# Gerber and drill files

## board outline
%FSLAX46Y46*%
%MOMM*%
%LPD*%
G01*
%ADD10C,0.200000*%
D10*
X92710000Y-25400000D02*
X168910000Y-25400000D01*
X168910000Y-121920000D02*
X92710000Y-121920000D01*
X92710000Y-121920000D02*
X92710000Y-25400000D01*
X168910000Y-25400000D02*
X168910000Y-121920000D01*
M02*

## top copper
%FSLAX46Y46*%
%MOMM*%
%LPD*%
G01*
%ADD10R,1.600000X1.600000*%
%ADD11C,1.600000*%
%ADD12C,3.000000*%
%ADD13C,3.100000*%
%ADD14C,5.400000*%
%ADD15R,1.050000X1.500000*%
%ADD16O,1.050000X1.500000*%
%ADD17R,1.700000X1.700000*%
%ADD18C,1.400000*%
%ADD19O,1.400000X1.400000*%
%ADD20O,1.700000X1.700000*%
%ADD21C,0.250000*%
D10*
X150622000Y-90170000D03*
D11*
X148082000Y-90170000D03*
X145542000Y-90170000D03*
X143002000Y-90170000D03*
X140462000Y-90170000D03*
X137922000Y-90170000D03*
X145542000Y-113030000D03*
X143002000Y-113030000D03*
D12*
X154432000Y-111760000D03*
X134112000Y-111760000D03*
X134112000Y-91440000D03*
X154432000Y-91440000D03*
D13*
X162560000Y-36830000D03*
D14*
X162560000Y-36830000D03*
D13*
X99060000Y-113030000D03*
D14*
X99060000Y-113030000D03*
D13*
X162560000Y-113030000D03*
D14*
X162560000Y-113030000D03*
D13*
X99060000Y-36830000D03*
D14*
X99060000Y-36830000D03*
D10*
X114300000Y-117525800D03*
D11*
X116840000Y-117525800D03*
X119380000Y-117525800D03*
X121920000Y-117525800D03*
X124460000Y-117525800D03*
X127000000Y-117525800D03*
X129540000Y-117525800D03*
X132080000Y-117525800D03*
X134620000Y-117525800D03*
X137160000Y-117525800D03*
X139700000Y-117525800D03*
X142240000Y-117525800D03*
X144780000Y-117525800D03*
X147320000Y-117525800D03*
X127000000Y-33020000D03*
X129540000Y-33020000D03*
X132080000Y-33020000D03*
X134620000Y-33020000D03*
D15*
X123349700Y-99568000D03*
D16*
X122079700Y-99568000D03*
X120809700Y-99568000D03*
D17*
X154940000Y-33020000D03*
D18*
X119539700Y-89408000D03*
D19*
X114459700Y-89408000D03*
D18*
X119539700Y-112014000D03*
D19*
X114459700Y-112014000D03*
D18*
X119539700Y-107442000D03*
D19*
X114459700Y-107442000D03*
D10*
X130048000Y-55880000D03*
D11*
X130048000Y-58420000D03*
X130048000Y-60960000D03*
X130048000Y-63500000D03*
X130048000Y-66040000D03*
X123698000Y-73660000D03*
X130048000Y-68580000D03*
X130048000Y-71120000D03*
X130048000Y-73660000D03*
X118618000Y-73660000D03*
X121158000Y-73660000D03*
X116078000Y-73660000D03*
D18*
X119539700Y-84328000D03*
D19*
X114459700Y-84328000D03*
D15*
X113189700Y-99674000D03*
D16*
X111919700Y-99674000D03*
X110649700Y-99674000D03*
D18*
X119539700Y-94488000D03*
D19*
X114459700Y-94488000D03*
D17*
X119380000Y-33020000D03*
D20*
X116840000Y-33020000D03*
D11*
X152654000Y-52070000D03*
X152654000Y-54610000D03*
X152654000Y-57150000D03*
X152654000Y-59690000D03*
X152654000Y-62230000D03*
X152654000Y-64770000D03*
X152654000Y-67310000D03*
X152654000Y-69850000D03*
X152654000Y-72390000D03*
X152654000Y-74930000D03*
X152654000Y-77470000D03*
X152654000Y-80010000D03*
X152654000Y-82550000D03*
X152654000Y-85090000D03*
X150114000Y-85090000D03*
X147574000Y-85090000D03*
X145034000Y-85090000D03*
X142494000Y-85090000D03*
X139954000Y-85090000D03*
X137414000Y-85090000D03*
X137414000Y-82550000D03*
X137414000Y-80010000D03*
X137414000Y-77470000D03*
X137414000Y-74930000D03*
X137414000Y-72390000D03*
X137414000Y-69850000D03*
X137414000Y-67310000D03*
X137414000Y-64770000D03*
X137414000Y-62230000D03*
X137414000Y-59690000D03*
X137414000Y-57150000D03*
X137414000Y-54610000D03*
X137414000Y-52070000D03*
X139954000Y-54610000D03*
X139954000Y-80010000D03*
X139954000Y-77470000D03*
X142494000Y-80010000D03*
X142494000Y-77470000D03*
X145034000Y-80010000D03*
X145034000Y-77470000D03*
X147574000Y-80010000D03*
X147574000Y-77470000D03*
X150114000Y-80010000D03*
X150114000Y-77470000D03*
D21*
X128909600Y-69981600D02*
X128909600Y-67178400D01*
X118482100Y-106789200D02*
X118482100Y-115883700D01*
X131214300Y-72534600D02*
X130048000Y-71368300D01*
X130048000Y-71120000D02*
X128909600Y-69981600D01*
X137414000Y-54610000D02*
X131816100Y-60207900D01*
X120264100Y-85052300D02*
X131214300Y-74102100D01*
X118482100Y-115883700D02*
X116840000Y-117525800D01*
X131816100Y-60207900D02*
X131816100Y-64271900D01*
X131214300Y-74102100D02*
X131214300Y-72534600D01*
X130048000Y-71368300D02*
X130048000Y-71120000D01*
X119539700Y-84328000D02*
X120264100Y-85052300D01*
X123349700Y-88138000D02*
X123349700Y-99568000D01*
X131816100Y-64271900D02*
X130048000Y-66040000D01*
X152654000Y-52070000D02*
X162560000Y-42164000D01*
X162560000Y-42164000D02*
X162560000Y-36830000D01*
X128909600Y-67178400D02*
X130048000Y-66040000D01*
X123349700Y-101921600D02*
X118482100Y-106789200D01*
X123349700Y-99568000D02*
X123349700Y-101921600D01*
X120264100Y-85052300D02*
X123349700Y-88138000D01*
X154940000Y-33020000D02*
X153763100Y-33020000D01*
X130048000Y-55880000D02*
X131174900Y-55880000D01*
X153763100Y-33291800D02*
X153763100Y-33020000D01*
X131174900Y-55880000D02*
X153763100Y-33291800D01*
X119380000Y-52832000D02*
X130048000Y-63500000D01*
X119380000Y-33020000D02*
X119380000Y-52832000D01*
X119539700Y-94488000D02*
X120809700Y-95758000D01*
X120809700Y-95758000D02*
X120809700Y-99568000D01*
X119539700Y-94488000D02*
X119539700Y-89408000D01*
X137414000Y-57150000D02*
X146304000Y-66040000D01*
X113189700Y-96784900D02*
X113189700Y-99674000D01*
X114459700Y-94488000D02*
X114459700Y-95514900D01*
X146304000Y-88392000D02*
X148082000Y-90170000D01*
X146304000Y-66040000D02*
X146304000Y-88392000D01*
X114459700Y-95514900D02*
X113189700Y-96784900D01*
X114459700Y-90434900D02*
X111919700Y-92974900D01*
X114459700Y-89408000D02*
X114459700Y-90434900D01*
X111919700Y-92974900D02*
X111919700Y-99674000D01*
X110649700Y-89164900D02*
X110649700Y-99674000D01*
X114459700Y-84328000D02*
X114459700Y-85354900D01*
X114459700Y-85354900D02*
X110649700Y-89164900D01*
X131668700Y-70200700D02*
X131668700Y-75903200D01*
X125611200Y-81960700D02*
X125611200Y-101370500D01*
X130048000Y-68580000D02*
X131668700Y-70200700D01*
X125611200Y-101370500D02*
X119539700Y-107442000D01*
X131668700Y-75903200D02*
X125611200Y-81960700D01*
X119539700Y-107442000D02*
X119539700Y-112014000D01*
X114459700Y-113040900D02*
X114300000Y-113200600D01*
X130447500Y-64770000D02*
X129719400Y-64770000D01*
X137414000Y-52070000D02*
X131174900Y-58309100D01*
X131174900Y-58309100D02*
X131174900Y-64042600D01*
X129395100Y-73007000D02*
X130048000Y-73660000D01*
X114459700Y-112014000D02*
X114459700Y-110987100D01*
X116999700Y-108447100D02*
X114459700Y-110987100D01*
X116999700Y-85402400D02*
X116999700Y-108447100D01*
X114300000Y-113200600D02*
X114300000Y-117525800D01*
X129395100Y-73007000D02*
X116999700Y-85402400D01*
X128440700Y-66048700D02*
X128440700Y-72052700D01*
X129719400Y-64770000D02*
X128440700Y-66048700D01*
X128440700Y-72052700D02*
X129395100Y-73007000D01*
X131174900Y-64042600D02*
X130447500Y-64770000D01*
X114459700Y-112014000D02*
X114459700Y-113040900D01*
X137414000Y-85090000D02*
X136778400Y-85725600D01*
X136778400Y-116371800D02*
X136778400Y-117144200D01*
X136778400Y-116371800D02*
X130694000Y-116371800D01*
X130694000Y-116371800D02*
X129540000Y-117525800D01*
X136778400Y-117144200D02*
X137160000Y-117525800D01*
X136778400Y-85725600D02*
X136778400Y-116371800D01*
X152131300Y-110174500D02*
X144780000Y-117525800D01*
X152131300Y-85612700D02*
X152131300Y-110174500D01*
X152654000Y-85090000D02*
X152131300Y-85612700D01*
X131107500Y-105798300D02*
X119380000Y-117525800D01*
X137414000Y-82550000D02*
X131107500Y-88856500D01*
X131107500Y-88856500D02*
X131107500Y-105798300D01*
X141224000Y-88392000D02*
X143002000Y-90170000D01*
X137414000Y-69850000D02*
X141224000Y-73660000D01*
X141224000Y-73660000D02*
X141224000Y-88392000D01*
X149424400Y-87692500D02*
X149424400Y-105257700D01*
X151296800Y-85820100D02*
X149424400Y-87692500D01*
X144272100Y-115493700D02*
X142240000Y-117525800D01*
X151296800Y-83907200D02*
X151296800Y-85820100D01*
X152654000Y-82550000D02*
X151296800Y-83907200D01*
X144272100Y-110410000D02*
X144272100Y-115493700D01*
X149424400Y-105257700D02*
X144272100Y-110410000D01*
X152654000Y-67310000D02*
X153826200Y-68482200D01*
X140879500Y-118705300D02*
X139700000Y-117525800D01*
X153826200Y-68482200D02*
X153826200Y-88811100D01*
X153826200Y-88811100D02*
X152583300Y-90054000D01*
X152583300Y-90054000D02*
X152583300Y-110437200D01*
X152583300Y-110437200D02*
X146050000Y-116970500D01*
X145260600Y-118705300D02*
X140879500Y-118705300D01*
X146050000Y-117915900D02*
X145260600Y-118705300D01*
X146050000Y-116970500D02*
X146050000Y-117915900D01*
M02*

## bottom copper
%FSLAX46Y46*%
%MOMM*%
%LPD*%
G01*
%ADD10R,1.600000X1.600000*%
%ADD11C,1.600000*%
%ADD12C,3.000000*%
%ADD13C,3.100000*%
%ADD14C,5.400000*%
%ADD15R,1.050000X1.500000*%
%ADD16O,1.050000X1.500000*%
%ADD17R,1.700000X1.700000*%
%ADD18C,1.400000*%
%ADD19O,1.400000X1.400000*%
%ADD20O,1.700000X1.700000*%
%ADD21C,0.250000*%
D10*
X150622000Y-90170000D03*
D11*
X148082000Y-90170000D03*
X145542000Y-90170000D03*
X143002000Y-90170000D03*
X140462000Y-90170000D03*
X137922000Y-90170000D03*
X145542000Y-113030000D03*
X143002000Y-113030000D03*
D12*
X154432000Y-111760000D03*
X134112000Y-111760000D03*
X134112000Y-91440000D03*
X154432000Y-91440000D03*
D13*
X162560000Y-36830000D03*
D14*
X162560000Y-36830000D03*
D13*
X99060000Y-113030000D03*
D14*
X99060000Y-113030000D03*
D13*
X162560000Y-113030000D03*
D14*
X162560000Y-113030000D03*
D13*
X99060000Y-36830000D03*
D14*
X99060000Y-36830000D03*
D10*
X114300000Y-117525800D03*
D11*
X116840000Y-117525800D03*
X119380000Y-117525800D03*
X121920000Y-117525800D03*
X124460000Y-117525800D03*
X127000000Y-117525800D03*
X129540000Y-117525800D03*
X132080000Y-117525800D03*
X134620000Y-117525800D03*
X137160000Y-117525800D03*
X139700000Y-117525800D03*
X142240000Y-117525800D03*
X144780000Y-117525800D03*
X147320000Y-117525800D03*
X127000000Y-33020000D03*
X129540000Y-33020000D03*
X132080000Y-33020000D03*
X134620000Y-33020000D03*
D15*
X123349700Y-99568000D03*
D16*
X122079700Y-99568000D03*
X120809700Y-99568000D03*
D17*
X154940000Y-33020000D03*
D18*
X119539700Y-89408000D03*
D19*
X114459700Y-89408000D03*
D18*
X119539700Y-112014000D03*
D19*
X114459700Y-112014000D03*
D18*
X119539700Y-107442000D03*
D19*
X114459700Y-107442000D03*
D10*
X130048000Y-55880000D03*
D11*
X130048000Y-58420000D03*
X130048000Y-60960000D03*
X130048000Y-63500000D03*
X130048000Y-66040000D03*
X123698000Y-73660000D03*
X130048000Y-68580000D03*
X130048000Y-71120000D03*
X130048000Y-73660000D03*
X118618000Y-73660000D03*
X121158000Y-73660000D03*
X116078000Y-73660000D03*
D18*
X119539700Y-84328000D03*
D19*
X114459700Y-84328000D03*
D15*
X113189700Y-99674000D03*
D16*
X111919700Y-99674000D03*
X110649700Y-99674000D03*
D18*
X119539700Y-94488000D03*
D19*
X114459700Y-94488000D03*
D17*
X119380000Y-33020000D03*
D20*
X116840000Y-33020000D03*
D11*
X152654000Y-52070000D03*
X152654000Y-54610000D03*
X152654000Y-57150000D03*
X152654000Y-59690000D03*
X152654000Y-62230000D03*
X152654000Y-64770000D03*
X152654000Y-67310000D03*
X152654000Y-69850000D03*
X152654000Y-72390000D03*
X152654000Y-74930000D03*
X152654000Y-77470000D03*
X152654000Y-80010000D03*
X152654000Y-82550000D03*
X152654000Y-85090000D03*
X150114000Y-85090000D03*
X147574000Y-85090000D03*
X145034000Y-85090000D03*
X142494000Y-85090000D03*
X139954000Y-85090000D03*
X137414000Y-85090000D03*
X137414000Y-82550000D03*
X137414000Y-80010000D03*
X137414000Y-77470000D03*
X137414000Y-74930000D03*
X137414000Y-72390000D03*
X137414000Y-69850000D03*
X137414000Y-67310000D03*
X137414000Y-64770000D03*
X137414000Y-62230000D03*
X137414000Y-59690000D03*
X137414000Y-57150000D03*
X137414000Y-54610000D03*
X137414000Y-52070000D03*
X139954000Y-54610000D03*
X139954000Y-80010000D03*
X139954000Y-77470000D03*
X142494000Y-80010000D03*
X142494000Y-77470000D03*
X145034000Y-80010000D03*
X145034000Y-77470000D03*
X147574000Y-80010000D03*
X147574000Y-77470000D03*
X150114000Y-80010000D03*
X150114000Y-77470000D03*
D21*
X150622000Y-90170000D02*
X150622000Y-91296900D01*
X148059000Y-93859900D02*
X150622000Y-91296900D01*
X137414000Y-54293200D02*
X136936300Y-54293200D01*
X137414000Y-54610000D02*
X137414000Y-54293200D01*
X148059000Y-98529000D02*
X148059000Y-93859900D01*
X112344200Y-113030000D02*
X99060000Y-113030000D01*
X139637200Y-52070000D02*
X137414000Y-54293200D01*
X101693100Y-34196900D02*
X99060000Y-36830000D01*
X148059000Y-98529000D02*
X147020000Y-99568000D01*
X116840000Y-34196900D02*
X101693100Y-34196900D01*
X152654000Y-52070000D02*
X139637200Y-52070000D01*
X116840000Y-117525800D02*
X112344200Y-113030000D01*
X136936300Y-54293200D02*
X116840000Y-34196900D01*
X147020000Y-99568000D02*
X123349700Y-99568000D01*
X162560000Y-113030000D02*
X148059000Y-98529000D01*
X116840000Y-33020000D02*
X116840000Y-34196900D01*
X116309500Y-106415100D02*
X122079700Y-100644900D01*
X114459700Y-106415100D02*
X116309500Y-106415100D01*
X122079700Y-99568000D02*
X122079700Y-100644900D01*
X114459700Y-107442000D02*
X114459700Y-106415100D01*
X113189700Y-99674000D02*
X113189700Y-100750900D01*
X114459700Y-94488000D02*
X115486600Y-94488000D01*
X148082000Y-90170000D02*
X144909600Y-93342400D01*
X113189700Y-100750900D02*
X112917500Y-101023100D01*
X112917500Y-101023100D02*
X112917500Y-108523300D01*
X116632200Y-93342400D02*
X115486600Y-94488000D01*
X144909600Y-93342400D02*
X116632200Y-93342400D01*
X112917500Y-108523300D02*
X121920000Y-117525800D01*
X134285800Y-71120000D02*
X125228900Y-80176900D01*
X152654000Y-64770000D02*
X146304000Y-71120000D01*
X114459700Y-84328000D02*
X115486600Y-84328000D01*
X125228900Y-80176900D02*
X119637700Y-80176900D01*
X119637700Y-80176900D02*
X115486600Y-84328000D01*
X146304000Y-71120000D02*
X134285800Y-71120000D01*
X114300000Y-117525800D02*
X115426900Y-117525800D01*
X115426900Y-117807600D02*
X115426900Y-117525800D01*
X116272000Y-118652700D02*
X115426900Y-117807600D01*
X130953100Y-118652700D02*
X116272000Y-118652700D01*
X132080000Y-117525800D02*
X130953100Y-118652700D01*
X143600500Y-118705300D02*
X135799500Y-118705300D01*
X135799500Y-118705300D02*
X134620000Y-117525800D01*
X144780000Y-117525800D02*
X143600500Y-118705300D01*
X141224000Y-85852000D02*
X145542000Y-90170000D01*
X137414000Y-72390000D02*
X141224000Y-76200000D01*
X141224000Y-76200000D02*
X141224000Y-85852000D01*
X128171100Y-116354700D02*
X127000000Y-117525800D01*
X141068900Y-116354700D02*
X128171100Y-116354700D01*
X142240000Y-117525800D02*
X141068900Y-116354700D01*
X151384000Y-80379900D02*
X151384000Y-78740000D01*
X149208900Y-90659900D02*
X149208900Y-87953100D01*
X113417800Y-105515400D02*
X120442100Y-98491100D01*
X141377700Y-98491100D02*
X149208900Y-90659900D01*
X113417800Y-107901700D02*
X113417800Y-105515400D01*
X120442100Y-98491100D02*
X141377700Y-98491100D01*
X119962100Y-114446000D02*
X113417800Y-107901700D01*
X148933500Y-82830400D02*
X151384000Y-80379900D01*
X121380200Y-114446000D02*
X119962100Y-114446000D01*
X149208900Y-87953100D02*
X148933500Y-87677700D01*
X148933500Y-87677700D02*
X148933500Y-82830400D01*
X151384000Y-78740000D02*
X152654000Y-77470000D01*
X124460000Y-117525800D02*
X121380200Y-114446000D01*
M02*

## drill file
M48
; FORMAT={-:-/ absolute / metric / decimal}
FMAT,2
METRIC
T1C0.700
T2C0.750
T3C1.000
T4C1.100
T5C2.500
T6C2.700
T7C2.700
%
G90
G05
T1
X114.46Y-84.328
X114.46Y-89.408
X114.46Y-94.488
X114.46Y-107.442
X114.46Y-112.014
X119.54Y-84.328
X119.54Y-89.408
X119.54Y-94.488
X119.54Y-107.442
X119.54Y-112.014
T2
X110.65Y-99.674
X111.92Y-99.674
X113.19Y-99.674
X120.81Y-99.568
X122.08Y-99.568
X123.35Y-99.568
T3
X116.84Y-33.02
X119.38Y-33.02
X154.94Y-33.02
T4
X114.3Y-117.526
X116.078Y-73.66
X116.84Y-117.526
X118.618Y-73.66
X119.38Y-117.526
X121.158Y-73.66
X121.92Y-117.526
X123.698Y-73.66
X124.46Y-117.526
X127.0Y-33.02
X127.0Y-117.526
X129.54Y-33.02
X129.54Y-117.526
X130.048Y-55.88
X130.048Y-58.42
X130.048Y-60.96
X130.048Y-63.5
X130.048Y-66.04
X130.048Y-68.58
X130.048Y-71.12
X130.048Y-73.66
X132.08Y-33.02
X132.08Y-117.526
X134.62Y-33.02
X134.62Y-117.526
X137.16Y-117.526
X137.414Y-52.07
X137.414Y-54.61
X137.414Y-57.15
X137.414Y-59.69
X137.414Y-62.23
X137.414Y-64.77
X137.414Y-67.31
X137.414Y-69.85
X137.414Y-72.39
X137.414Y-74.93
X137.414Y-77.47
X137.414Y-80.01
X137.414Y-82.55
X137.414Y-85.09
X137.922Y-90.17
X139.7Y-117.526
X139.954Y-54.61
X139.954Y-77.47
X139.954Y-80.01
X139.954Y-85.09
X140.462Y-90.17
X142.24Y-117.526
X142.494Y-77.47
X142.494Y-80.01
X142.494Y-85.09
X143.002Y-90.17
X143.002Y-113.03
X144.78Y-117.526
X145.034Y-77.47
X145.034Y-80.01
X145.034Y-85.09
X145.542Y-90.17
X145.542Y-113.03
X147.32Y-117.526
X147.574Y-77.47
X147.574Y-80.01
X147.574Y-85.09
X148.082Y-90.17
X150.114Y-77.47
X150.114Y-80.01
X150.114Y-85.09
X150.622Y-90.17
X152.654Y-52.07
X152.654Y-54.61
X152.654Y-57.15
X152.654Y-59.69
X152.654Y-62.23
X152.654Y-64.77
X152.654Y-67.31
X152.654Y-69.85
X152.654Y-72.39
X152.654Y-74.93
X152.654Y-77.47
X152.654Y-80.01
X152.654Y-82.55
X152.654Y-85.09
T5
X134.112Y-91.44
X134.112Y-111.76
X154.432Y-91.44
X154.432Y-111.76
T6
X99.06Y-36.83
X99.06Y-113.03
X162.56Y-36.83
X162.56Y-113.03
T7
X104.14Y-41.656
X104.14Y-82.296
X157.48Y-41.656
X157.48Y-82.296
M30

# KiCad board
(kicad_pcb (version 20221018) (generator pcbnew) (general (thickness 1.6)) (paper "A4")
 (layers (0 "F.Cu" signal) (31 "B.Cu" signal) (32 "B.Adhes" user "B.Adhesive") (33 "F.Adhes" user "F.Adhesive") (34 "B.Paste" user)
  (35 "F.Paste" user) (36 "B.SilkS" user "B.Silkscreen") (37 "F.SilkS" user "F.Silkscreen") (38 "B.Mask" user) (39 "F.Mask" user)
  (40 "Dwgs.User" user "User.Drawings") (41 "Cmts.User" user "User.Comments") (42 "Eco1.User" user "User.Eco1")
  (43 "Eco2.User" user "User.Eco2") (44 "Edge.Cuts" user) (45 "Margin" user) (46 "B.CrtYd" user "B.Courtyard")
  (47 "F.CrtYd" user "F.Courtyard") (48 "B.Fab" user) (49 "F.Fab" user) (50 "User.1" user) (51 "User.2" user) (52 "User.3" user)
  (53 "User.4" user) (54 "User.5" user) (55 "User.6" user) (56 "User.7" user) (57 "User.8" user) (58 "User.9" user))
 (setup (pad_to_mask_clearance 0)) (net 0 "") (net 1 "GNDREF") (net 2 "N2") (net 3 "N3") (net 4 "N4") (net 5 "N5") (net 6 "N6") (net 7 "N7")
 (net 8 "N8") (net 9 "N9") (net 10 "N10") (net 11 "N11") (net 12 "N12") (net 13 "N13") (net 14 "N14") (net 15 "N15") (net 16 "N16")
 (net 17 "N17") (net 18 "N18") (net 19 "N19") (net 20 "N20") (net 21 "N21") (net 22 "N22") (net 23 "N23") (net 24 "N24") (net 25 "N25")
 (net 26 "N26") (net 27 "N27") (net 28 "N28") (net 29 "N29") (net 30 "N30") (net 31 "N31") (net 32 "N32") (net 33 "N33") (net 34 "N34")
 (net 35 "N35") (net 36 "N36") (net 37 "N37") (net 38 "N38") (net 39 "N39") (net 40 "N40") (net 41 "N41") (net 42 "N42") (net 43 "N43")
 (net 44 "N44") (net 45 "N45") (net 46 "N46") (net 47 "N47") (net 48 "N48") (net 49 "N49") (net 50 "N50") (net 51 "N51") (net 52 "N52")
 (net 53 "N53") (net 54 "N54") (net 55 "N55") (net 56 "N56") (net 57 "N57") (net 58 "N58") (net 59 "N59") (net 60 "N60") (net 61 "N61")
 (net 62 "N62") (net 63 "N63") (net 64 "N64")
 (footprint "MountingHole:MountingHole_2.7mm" (layer "F.Cu") (at 157.48 41.656)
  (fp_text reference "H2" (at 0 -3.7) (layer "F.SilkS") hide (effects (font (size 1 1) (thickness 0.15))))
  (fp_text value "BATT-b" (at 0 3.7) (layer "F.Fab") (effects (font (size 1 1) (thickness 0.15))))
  (pad "" np_thru_hole circle (at 0 0) (size 2.7 2.7) (drill 2.7) (layers "*.Cu" "*.Mask")))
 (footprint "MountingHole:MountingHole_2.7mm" (layer "F.Cu") (at 157.48 82.296)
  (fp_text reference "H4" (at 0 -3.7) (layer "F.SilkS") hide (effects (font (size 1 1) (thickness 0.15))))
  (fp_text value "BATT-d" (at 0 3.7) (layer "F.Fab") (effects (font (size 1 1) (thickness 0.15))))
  (pad "" np_thru_hole circle (at 0 0) (size 2.7 2.7) (drill 2.7) (layers "*.Cu" "*.Mask")))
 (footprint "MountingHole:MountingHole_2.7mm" (layer "F.Cu") (at 104.14 82.296)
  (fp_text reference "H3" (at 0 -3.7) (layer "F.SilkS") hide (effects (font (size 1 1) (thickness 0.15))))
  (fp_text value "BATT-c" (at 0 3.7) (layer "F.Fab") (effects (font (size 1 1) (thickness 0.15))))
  (pad "" np_thru_hole circle (at 0 0) (size 2.7 2.7) (drill 2.7) (layers "*.Cu" "*.Mask")))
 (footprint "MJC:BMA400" (layer "F.Cu") (at 144.272 101.6 180)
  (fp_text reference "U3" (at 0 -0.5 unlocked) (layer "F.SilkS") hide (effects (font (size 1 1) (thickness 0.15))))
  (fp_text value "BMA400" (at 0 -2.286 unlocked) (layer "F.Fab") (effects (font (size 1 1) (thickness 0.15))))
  (pad "1" thru_hole rect (at -6.35 11.43 180) (size 1.6 1.6) (drill 1.1) (layers "*.Cu" "*.Mask") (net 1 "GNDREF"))
  (pad "2" thru_hole circle (at -3.81 11.43 180) (size 1.6 1.6) (drill 1.1) (layers "*.Cu" "*.Mask") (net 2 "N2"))
  (pad "3" thru_hole circle (at -1.27 11.43 180) (size 1.6 1.6) (drill 1.1) (layers "*.Cu" "*.Mask") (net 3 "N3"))
  (pad "4" thru_hole circle (at 1.27 11.43 180) (size 1.6 1.6) (drill 1.1) (layers "*.Cu" "*.Mask") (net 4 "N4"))
  (pad "5" thru_hole circle (at 3.81 11.43 180) (size 1.6 1.6) (drill 1.1) (layers "*.Cu" "*.Mask") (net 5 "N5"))
  (pad "6" thru_hole circle (at 6.35 11.43 180) (size 1.6 1.6) (drill 1.1) (layers "*.Cu" "*.Mask") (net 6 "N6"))
  (pad "7" thru_hole circle (at -1.27 -11.43 180) (size 1.6 1.6) (drill 1.1) (layers "*.Cu" "*.Mask") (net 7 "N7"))
  (pad "8" thru_hole circle (at 1.27 -11.43 180) (size 1.6 1.6) (drill 1.1) (layers "*.Cu" "*.Mask") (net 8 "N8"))
  (pad "9" thru_hole circle (at -10.16 -10.16 180) (size 3 3) (drill 2.5) (layers "*.Cu" "*.Mask"))
  (pad "10" thru_hole circle (at 10.16 -10.16 180) (size 3 3) (drill 2.5) (layers "*.Cu" "*.Mask"))
  (pad "11" thru_hole circle (at 10.16 10.16 180) (size 3 3) (drill 2.5) (layers "*.Cu" "*.Mask"))
  (pad "12" thru_hole circle (at -10.16 10.16 180) (size 3 3) (drill 2.5) (layers "*.Cu" "*.Mask")))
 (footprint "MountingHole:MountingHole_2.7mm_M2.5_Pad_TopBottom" (layer "F.Cu") (at 162.56 36.83)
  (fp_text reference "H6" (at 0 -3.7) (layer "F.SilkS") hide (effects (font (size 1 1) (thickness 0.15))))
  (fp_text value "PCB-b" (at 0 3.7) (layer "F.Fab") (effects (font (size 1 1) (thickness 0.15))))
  (pad "1" thru_hole circle (at 0 0) (size 3.1 3.1) (drill 2.7) (layers "*.Cu" "*.Mask") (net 1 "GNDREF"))
  (pad "1" connect circle (at 0 0) (size 5.4 5.4) (layers "F.Cu" "F.Mask") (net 1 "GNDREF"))
  (pad "1" connect circle (at 0 0) (size 5.4 5.4) (layers "B.Cu" "B.Mask") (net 1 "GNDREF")))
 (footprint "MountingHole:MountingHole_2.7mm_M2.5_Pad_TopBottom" (layer "F.Cu") (at 99.06 113.03)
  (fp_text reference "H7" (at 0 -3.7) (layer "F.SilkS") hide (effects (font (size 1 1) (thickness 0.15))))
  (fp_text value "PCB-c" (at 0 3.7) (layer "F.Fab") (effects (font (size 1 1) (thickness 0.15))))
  (pad "1" thru_hole circle (at 0 0) (size 3.1 3.1) (drill 2.7) (layers "*.Cu" "*.Mask") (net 1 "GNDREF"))
  (pad "1" connect circle (at 0 0) (size 5.4 5.4) (layers "F.Cu" "F.Mask") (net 1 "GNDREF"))
  (pad "1" connect circle (at 0 0) (size 5.4 5.4) (layers "B.Cu" "B.Mask") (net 1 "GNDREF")))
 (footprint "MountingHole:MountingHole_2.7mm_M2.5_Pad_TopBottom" (layer "F.Cu") (at 162.56 113.03)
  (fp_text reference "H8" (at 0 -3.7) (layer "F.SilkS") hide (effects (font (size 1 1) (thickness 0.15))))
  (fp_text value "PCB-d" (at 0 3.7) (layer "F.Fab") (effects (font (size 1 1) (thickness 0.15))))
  (pad "1" thru_hole circle (at 0 0) (size 3.1 3.1) (drill 2.7) (layers "*.Cu" "*.Mask") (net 1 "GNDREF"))
  (pad "1" connect circle (at 0 0) (size 5.4 5.4) (layers "F.Cu" "F.Mask") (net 1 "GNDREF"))
  (pad "1" connect circle (at 0 0) (size 5.4 5.4) (layers "B.Cu" "B.Mask") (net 1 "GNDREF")))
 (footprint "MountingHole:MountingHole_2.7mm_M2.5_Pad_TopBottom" (layer "F.Cu") (at 99.06 36.83)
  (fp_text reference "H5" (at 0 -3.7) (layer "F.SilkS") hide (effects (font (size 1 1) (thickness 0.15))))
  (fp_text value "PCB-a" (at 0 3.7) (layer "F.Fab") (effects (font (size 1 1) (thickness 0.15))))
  (pad "1" thru_hole circle (at 0 0) (size 3.1 3.1) (drill 2.7) (layers "*.Cu" "*.Mask") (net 1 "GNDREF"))
  (pad "1" connect circle (at 0 0) (size 5.4 5.4) (layers "F.Cu" "F.Mask") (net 1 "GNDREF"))
  (pad "1" connect circle (at 0 0) (size 5.4 5.4) (layers "B.Cu" "B.Mask") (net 1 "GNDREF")))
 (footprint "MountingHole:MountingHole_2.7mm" (layer "F.Cu") (at 104.14 41.656)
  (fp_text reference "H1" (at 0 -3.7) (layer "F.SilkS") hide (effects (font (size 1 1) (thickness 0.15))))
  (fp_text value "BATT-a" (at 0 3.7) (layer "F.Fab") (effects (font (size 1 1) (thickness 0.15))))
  (pad "" np_thru_hole circle (at 0 0) (size 2.7 2.7) (drill 2.7) (layers "*.Cu" "*.Mask")))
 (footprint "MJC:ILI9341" (layer "F.Cu") (at 130.81 74.7776)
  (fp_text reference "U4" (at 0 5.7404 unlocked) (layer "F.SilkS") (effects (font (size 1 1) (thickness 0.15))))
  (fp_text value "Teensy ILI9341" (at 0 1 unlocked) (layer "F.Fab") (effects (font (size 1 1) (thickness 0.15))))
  (pad "1" thru_hole rect (at -16.51 42.7482) (size 1.6 1.6) (drill 1.1) (layers "*.Cu" "*.Mask") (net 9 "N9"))
  (pad "2" thru_hole circle (at -13.97 42.7482) (size 1.6 1.6) (drill 1.1) (layers "*.Cu" "*.Mask") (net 1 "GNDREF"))
  (pad "3" thru_hole circle (at -11.43 42.7482) (size 1.6 1.6) (drill 1.1) (layers "*.Cu" "*.Mask") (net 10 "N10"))
  (pad "4" thru_hole circle (at -8.89 42.7482) (size 1.6 1.6) (drill 1.1) (layers "*.Cu" "*.Mask") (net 2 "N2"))
  (pad "5" thru_hole circle (at -6.35 42.7482) (size 1.6 1.6) (drill 1.1) (layers "*.Cu" "*.Mask") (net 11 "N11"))
  (pad "6" thru_hole circle (at -3.81 42.7482) (size 1.6 1.6) (drill 1.1) (layers "*.Cu" "*.Mask") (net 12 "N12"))
  (pad "7" thru_hole circle (at -1.27 42.7482) (size 1.6 1.6) (drill 1.1) (layers "*.Cu" "*.Mask") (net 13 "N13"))
  (pad "8" thru_hole circle (at 1.27 42.7482) (size 1.6 1.6) (drill 1.1) (layers "*.Cu" "*.Mask") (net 9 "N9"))
  (pad "9" thru_hole circle (at 3.81 42.7482) (size 1.6 1.6) (drill 1.1) (layers "*.Cu" "*.Mask") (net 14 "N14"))
  (pad "10" thru_hole circle (at 6.35 42.7482) (size 1.6 1.6) (drill 1.1) (layers "*.Cu" "*.Mask") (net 13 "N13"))
  (pad "11" thru_hole circle (at 8.89 42.7482) (size 1.6 1.6) (drill 1.1) (layers "*.Cu" "*.Mask") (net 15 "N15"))
  (pad "12" thru_hole circle (at 11.43 42.7482) (size 1.6 1.6) (drill 1.1) (layers "*.Cu" "*.Mask") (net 12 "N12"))
  (pad "13" thru_hole circle (at 13.97 42.7482) (size 1.6 1.6) (drill 1.1) (layers "*.Cu" "*.Mask") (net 14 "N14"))
  (pad "14" thru_hole circle (at 16.51 42.7482) (size 1.6 1.6) (drill 1.1) (layers "*.Cu" "*.Mask") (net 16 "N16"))
  (pad "15" thru_hole circle (at -3.81 -41.7576) (size 1.6 1.6) (drill 1.1) (layers "*.Cu" "*.Mask") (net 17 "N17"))
  (pad "16" thru_hole circle (at -1.27 -41.7576) (size 1.6 1.6) (drill 1.1) (layers "*.Cu" "*.Mask") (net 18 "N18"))
  (pad "17" thru_hole circle (at 1.27 -41.7576) (size 1.6 1.6) (drill 1.1) (layers "*.Cu" "*.Mask") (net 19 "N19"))
  (pad "18" thru_hole circle (at 3.81 -41.7576) (size 1.6 1.6) (drill 1.1) (layers "*.Cu" "*.Mask") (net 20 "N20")))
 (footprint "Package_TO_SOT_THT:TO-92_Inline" (layer "B.Cu") (at 123.3497 99.568 180)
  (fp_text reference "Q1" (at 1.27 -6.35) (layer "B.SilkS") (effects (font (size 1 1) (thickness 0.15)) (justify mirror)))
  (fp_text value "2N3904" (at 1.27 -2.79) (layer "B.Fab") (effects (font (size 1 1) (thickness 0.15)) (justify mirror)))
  (pad "1" thru_hole rect (at 0 0 180) (size 1.05 1.5) (drill 0.75) (layers "*.Cu" "*.Mask") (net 1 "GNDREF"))
  (pad "2" thru_hole oval (at 1.27 0 180) (size 1.05 1.5) (drill 0.75) (layers "*.Cu" "*.Mask") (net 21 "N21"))
  (pad "3" thru_hole oval (at 2.54 0 180) (size 1.05 1.5) (drill 0.75) (layers "*.Cu" "*.Mask") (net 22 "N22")))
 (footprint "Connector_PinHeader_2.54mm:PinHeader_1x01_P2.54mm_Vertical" (layer "B.Cu") (at 154.94 33.02 180)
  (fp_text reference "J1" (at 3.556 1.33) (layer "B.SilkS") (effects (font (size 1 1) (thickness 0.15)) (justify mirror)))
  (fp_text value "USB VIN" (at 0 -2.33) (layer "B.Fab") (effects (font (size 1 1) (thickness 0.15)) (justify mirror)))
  (pad "1" thru_hole rect (at 0 0 180) (size 1.7 1.7) (drill 1) (layers "*.Cu" "*.Mask") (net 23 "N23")))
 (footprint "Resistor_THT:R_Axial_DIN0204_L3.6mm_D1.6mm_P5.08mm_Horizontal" (layer "B.Cu") (at 119.5397 89.408 180)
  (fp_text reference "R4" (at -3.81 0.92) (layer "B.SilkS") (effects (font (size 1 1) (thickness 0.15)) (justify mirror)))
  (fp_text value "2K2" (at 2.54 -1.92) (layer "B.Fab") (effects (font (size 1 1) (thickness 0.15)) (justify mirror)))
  (pad "1" thru_hole circle (at 0 0 180) (size 1.4 1.4) (drill 0.7) (layers "*.Cu" "*.Mask") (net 22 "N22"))
  (pad "2" thru_hole oval (at 5.08 0 180) (size 1.4 1.4) (drill 0.7) (layers "*.Cu" "*.Mask") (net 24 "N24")))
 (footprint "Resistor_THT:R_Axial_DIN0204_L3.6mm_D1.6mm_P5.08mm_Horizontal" (layer "B.Cu") (at 119.5397 112.014 180)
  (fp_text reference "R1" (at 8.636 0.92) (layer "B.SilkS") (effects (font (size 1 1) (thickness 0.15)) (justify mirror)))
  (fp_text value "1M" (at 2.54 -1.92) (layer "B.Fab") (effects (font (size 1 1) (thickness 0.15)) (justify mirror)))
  (pad "1" thru_hole circle (at 0 0 180) (size 1.4 1.4) (drill 0.7) (layers "*.Cu" "*.Mask") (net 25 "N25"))
  (pad "2" thru_hole oval (at 5.08 0 180) (size 1.4 1.4) (drill 0.7) (layers "*.Cu" "*.Mask") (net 9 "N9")))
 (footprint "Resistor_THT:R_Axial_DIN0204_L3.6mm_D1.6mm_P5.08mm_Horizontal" (layer "B.Cu") (at 119.5397 107.442 180)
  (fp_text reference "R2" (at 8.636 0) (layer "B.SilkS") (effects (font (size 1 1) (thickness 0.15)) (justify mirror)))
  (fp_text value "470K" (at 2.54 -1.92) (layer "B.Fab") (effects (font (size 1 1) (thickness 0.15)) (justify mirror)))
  (pad "1" thru_hole circle (at 0 0 180) (size 1.4 1.4) (drill 0.7) (layers "*.Cu" "*.Mask") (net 25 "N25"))
  (pad "2" thru_hole oval (at 5.08 0 180) (size 1.4 1.4) (drill 0.7) (layers "*.Cu" "*.Mask") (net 21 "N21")))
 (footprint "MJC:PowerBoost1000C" (layer "B.Cu") (at 119.888 60.96 180)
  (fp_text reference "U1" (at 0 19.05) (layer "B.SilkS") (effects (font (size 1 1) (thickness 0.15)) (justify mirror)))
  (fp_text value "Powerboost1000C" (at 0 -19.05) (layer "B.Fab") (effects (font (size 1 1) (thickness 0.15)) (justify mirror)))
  (pad "1" thru_hole rect (at -10.16 5.08 180) (size 1.6 1.6) (drill 1.1) (layers "*.Cu" "*.Mask") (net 23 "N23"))
  (pad "2" thru_hole circle (at -10.16 2.54 180) (size 1.6 1.6) (drill 1.1) (layers "*.Cu" "*.Mask") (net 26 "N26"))
  (pad "3" thru_hole circle (at -10.16 0 180) (size 1.6 1.6) (drill 1.1) (layers "*.Cu" "*.Mask") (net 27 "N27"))
  (pad "4" thru_hole circle (at -10.16 -2.54 180) (size 1.6 1.6) (drill 1.1) (layers "*.Cu" "*.Mask") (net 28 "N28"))
  (pad "5" thru_hole circle (at -10.16 -5.08 180) (size 1.6 1.6) (drill 1.1) (layers "*.Cu" "*.Mask") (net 1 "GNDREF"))
  (pad "5V" thru_hole circle (at -3.81 -12.7 180) (size 1.6 1.6) (drill 1.1) (layers "*.Cu" "*.Mask") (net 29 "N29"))
  (pad "6" thru_hole circle (at -10.16 -7.62 180) (size 1.6 1.6) (drill 1.1) (layers "*.Cu" "*.Mask") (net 25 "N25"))
  (pad "7" thru_hole circle (at -10.16 -10.16 180) (size 1.6 1.6) (drill 1.1) (layers "*.Cu" "*.Mask") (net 1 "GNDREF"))
  (pad "8" thru_hole circle (at -10.16 -12.7 180) (size 1.6 1.6) (drill 1.1) (layers "*.Cu" "*.Mask") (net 9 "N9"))
  (pad "D+" thru_hole circle (at 1.27 -12.7 180) (size 1.6 1.6) (drill 1.1) (layers "*.Cu" "*.Mask") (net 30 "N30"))
  (pad "D-" thru_hole circle (at -1.27 -12.7 180) (size 1.6 1.6) (drill 1.1) (layers "*.Cu" "*.Mask") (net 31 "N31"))
  (pad "UG" thru_hole circle (at 3.81 -12.7 180) (size 1.6 1.6) (drill 1.1) (layers "*.Cu" "*.Mask") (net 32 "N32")))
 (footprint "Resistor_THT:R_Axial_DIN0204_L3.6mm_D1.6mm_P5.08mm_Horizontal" (layer "B.Cu") (at 119.5397 84.328 180)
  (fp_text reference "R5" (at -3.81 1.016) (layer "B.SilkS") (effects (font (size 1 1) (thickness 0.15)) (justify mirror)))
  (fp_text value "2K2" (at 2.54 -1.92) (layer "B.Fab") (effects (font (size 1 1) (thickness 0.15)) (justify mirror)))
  (pad "1" thru_hole circle (at 0 0 180) (size 1.4 1.4) (drill 0.7) (layers "*.Cu" "*.Mask") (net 1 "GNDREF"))
  (pad "2" thru_hole oval (at 5.08 0 180) (size 1.4 1.4) (drill 0.7) (layers "*.Cu" "*.Mask") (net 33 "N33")))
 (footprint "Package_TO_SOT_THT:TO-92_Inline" (layer "B.Cu") (at 113.1897 99.674 180)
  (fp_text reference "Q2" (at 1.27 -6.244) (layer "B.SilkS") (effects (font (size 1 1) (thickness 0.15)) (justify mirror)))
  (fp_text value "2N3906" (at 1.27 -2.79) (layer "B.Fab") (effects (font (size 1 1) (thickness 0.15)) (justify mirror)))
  (pad "1" thru_hole rect (at 0 0 180) (size 1.05 1.5) (drill 0.75) (layers "*.Cu" "*.Mask") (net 2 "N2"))
  (pad "2" thru_hole oval (at 1.27 0 180) (size 1.05 1.5) (drill 0.75) (layers "*.Cu" "*.Mask") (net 24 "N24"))
  (pad "3" thru_hole oval (at 2.54 0 180) (size 1.05 1.5) (drill 0.75) (layers "*.Cu" "*.Mask") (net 33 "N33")))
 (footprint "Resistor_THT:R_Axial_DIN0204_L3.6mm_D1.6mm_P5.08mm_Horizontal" (layer "B.Cu") (at 119.5397 94.488 180)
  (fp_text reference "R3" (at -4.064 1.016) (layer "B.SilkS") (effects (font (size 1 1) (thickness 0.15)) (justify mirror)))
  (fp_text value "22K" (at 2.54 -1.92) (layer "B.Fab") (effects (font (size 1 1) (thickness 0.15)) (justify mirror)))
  (pad "1" thru_hole circle (at 0 0 180) (size 1.4 1.4) (drill 0.7) (layers "*.Cu" "*.Mask") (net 22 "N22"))
  (pad "2" thru_hole oval (at 5.08 0 180) (size 1.4 1.4) (drill 0.7) (layers "*.Cu" "*.Mask") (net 2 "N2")))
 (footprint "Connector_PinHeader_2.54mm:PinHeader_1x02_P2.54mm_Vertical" (layer "B.Cu") (at 119.38 33.02 90)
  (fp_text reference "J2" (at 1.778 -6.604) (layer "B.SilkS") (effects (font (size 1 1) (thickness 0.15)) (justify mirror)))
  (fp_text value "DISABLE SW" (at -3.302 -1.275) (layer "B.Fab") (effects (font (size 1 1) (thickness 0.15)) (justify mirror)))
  (pad "1" thru_hole rect (at 0 0 90) (size 1.7 1.7) (drill 1) (layers "*.Cu" "*.Mask") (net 28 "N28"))
  (pad "2" thru_hole oval (at 0 -2.54 90) (size 1.7 1.7) (drill 1) (layers "*.Cu" "*.Mask") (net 1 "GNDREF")))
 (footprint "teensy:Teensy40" (layer "B.Cu") (at 145.034 68.58 -90)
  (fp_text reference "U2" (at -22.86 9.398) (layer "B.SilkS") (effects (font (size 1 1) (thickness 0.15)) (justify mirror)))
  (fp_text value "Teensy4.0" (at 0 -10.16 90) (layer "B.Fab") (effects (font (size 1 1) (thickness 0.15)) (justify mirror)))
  (pad "1" thru_hole circle (at -16.51 -7.62 270) (size 1.6 1.6) (drill 1.1) (layers "*.Cu" "*.Mask") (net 1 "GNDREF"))
  (pad "2" thru_hole circle (at -13.97 -7.62 270) (size 1.6 1.6) (drill 1.1) (layers "*.Cu" "*.Mask") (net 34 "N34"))
  (pad "3" thru_hole circle (at -11.43 -7.62 270) (size 1.6 1.6) (drill 1.1) (layers "*.Cu" "*.Mask") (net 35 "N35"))
  (pad "4" thru_hole circle (at -8.89 -7.62 270) (size 1.6 1.6) (drill 1.1) (layers "*.Cu" "*.Mask") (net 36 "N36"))
  (pad "5" thru_hole circle (at -6.35 -7.62 270) (size 1.6 1.6) (drill 1.1) (layers "*.Cu" "*.Mask") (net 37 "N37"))
  (pad "6" thru_hole circle (at -3.81 -7.62 270) (size 1.6 1.6) (drill 1.1) (layers "*.Cu" "*.Mask") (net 33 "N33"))
  (pad "7" thru_hole circle (at -1.27 -7.62 270) (size 1.6 1.6) (drill 1.1) (layers "*.Cu" "*.Mask") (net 15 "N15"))
  (pad "8" thru_hole circle (at 1.27 -7.62 270) (size 1.6 1.6) (drill 1.1) (layers "*.Cu" "*.Mask") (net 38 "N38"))
  (pad "9" thru_hole circle (at 3.81 -7.62 270) (size 1.6 1.6) (drill 1.1) (layers "*.Cu" "*.Mask") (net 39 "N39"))
  (pad "10" thru_hole circle (at 6.35 -7.62 270) (size 1.6 1.6) (drill 1.1) (layers "*.Cu" "*.Mask") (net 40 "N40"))
  (pad "11" thru_hole circle (at 8.89 -7.62 270) (size 1.6 1.6) (drill 1.1) (layers "*.Cu" "*.Mask") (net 11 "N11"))
  (pad "12" thru_hole circle (at 11.43 -7.62 270) (size 1.6 1.6) (drill 1.1) (layers "*.Cu" "*.Mask") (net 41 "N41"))
  (pad "13" thru_hole circle (at 13.97 -7.62 270) (size 1.6 1.6) (drill 1.1) (layers "*.Cu" "*.Mask") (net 12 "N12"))
  (pad "14" thru_hole circle (at 16.51 -7.62 270) (size 1.6 1.6) (drill 1.1) (layers "*.Cu" "*.Mask") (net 14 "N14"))
  (pad "15" thru_hole circle (at 16.51 -5.08 270) (size 1.6 1.6) (drill 1.1) (layers "*.Cu" "*.Mask") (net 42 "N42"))
  (pad "16" thru_hole circle (at 16.51 -2.54 270) (size 1.6 1.6) (drill 1.1) (layers "*.Cu" "*.Mask") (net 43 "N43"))
  (pad "17" thru_hole circle (at 16.51 0 270) (size 1.6 1.6) (drill 1.1) (layers "*.Cu" "*.Mask") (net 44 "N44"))
  (pad "18" thru_hole circle (at 16.51 2.54 270) (size 1.6 1.6) (drill 1.1) (layers "*.Cu" "*.Mask") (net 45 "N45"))
  (pad "19" thru_hole circle (at 16.51 5.08 270) (size 1.6 1.6) (drill 1.1) (layers "*.Cu" "*.Mask") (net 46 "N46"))
  (pad "20" thru_hole circle (at 16.51 7.62 270) (size 1.6 1.6) (drill 1.1) (layers "*.Cu" "*.Mask") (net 13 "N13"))
  (pad "21" thru_hole circle (at 13.97 7.62 270) (size 1.6 1.6) (drill 1.1) (layers "*.Cu" "*.Mask") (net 10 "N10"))
  (pad "22" thru_hole circle (at 11.43 7.62 270) (size 1.6 1.6) (drill 1.1) (layers "*.Cu" "*.Mask") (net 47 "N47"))
  (pad "23" thru_hole circle (at 8.89 7.62 270) (size 1.6 1.6) (drill 1.1) (layers "*.Cu" "*.Mask") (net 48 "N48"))
  (pad "24" thru_hole circle (at 6.35 7.62 270) (size 1.6 1.6) (drill 1.1) (layers "*.Cu" "*.Mask") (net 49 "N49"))
  (pad "25" thru_hole circle (at 3.81 7.62 270) (size 1.6 1.6) (drill 1.1) (layers "*.Cu" "*.Mask") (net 3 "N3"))
  (pad "26" thru_hole circle (at 1.27 7.62 270) (size 1.6 1.6) (drill 1.1) (layers "*.Cu" "*.Mask") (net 4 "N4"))
  (pad "27" thru_hole circle (at -1.27 7.62 270) (size 1.6 1.6) (drill 1.1) (layers "*.Cu" "*.Mask") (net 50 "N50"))
  (pad "28" thru_hole circle (at -3.81 7.62 270) (size 1.6 1.6) (drill 1.1) (layers "*.Cu" "*.Mask") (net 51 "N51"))
  (pad "29" thru_hole circle (at -6.35 7.62 270) (size 1.6 1.6) (drill 1.1) (layers "*.Cu" "*.Mask") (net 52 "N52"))
  (pad "30" thru_hole circle (at -8.89 7.62 270) (size 1.6 1.6) (drill 1.1) (layers "*.Cu" "*.Mask") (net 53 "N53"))
  (pad "31" thru_hole circle (at -11.43 7.62 270) (size 1.6 1.6) (drill 1.1) (layers "*.Cu" "*.Mask") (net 2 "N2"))
  (pad "32" thru_hole circle (at -13.97 7.62 270) (size 1.6 1.6) (drill 1.1) (layers "*.Cu" "*.Mask") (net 1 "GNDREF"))
  (pad "33" thru_hole circle (at -16.51 7.62 270) (size 1.6 1.6) (drill 1.1) (layers "*.Cu" "*.Mask") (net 9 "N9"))
  (pad "34" thru_hole circle (at -13.97 5.08 270) (size 1.6 1.6) (drill 1.1) (layers "*.Cu" "*.Mask") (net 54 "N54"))
  (pad "35" thru_hole circle (at 11.43 5.08 270) (size 1.6 1.6) (drill 1.1) (layers "*.Cu" "*.Mask") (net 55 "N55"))
  (pad "36" thru_hole circle (at 8.89 5.08 270) (size 1.6 1.6) (drill 1.1) (layers "*.Cu" "*.Mask") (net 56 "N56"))
  (pad "37" thru_hole circle (at 11.43 2.54 270) (size 1.6 1.6) (drill 1.1) (layers "*.Cu" "*.Mask") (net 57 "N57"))
  (pad "38" thru_hole circle (at 8.89 2.54 270) (size 1.6 1.6) (drill 1.1) (layers "*.Cu" "*.Mask") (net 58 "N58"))
  (pad "39" thru_hole circle (at 11.43 0 270) (size 1.6 1.6) (drill 1.1) (layers "*.Cu" "*.Mask") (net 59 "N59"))
  (pad "40" thru_hole circle (at 8.89 0 270) (size 1.6 1.6) (drill 1.1) (layers "*.Cu" "*.Mask") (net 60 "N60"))
  (pad "41" thru_hole circle (at 11.43 -2.54 270) (size 1.6 1.6) (drill 1.1) (layers "*.Cu" "*.Mask") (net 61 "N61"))
  (pad "42" thru_hole circle (at 8.89 -2.54 270) (size 1.6 1.6) (drill 1.1) (layers "*.Cu" "*.Mask") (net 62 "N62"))
  (pad "43" thru_hole circle (at 11.43 -5.08 270) (size 1.6 1.6) (drill 1.1) (layers "*.Cu" "*.Mask") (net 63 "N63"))
  (pad "44" thru_hole circle (at 8.89 -5.08 270) (size 1.6 1.6) (drill 1.1) (layers "*.Cu" "*.Mask") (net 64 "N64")))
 (gr_line (start 92.71 25.4) (end 168.91 25.4) (stroke (width 0.2) (type default)) (layer "Edge.Cuts"))
 (gr_line (start 168.91 121.92) (end 92.71 121.92) (stroke (width 0.2) (type default)) (layer "Edge.Cuts"))
 (gr_line (start 92.71 121.92) (end 92.71 25.4) (stroke (width 0.2) (type default)) (layer "Edge.Cuts"))
 (gr_line (start 168.91 25.4) (end 168.91 121.92) (stroke (width 0.2) (type default)) (layer "Edge.Cuts"))
 (segment (start 128.9096 69.9816) (end 128.9096 67.1784) (width 0.25) (layer "F.Cu") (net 1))
 (segment (start 118.4821 106.7892) (end 118.4821 115.8837) (width 0.25) (layer "F.Cu") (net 1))
 (segment (start 131.2143 72.5346) (end 130.048 71.3683) (width 0.25) (layer "F.Cu") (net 1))
 (segment (start 130.048 71.12) (end 128.9096 69.9816) (width 0.25) (layer "F.Cu") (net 1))
 (segment (start 137.414 54.61) (end 131.8161 60.2079) (width 0.25) (layer "F.Cu") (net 1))
 (segment (start 120.2641 85.0523) (end 131.2143 74.1021) (width 0.25) (layer "F.Cu") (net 1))
 (segment (start 118.4821 115.8837) (end 116.84 117.5258) (width 0.25) (layer "F.Cu") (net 1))
 (segment (start 131.8161 60.2079) (end 131.8161 64.2719) (width 0.25) (layer "F.Cu") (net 1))
 (segment (start 131.2143 74.1021) (end 131.2143 72.5346) (width 0.25) (layer "F.Cu") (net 1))
 (segment (start 130.048 71.3683) (end 130.048 71.12) (width 0.25) (layer "F.Cu") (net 1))
 (segment (start 119.5397 84.328) (end 120.2641 85.0523) (width 0.25) (layer "F.Cu") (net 1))
 (segment (start 123.3497 88.138) (end 123.3497 99.568) (width 0.25) (layer "F.Cu") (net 1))
 (segment (start 131.8161 64.2719) (end 130.048 66.04) (width 0.25) (layer "F.Cu") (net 1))
 (segment (start 152.654 52.07) (end 162.56 42.164) (width 0.25) (layer "F.Cu") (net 1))
 (segment (start 162.56 42.164) (end 162.56 36.83) (width 0.25) (layer "F.Cu") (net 1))
 (segment (start 128.9096 67.1784) (end 130.048 66.04) (width 0.25) (layer "F.Cu") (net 1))
 (segment (start 123.3497 101.9216) (end 118.4821 106.7892) (width 0.25) (layer "F.Cu") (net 1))
 (segment (start 123.3497 99.568) (end 123.3497 101.9216) (width 0.25) (layer "F.Cu") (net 1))
 (segment (start 120.2641 85.0523) (end 123.3497 88.138) (width 0.25) (layer "F.Cu") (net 1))
 (segment (start 150.622 90.17) (end 150.622 91.2969) (width 0.25) (layer "B.Cu") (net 1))
 (segment (start 148.059 93.8599) (end 150.622 91.2969) (width 0.25) (layer "B.Cu") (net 1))
 (segment (start 137.414 54.2932) (end 136.9363 54.2932) (width 0.25) (layer "B.Cu") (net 1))
 (segment (start 137.414 54.61) (end 137.414 54.2932) (width 0.25) (layer "B.Cu") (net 1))
 (segment (start 148.059 98.529) (end 148.059 93.8599) (width 0.25) (layer "B.Cu") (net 1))
 (segment (start 112.3442 113.03) (end 99.06 113.03) (width 0.25) (layer "B.Cu") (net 1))
 (segment (start 139.6372 52.07) (end 137.414 54.2932) (width 0.25) (layer "B.Cu") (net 1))
 (segment (start 101.6931 34.1969) (end 99.06 36.83) (width 0.25) (layer "B.Cu") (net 1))
 (segment (start 148.059 98.529) (end 147.02 99.568) (width 0.25) (layer "B.Cu") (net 1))
 (segment (start 116.84 34.1969) (end 101.6931 34.1969) (width 0.25) (layer "B.Cu") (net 1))
 (segment (start 152.654 52.07) (end 139.6372 52.07) (width 0.25) (layer "B.Cu") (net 1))
 (segment (start 116.84 117.5258) (end 112.3442 113.03) (width 0.25) (layer "B.Cu") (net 1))
 (segment (start 136.9363 54.2932) (end 116.84 34.1969) (width 0.25) (layer "B.Cu") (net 1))
 (segment (start 147.02 99.568) (end 123.3497 99.568) (width 0.25) (layer "B.Cu") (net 1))
 (segment (start 162.56 113.03) (end 148.059 98.529) (width 0.25) (layer "B.Cu") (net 1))
 (segment (start 116.84 33.02) (end 116.84 34.1969) (width 0.25) (layer "B.Cu") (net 1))
 (segment (start 154.94 33.02) (end 153.7631 33.02) (width 0.25) (layer "F.Cu") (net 23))
 (segment (start 130.048 55.88) (end 131.1749 55.88) (width 0.25) (layer "F.Cu") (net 23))
 (segment (start 153.7631 33.2918) (end 153.7631 33.02) (width 0.25) (layer "F.Cu") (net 23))
 (segment (start 131.1749 55.88) (end 153.7631 33.2918) (width 0.25) (layer "F.Cu") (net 23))
 (segment (start 119.38 52.832) (end 130.048 63.5) (width 0.25) (layer "F.Cu") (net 28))
 (segment (start 119.38 33.02) (end 119.38 52.832) (width 0.25) (layer "F.Cu") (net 28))
 (segment (start 116.3095 106.4151) (end 122.0797 100.6449) (width 0.25) (layer "B.Cu") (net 21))
 (segment (start 114.4597 106.4151) (end 116.3095 106.4151) (width 0.25) (layer "B.Cu") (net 21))
 (segment (start 122.0797 99.568) (end 122.0797 100.6449) (width 0.25) (layer "B.Cu") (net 21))
 (segment (start 114.4597 107.442) (end 114.4597 106.4151) (width 0.25) (layer "B.Cu") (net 21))
 (segment (start 119.5397 94.488) (end 120.8097 95.758) (width 0.25) (layer "F.Cu") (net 22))
 (segment (start 120.8097 95.758) (end 120.8097 99.568) (width 0.25) (layer "F.Cu") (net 22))
 (segment (start 119.5397 94.488) (end 119.5397 89.408) (width 0.25) (layer "F.Cu") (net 22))
 (segment (start 137.414 57.15) (end 146.304 66.04) (width 0.25) (layer "F.Cu") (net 2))
 (segment (start 113.1897 96.7849) (end 113.1897 99.674) (width 0.25) (layer "F.Cu") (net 2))
 (segment (start 114.4597 94.488) (end 114.4597 95.5149) (width 0.25) (layer "F.Cu") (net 2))
 (segment (start 146.304 88.392) (end 148.082 90.17) (width 0.25) (layer "F.Cu") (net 2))
 (segment (start 146.304 66.04) (end 146.304 88.392) (width 0.25) (layer "F.Cu") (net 2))
 (segment (start 114.4597 95.5149) (end 113.1897 96.7849) (width 0.25) (layer "F.Cu") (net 2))
 (segment (start 113.1897 99.674) (end 113.1897 100.7509) (width 0.25) (layer "B.Cu") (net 2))
 (segment (start 114.4597 94.488) (end 115.4866 94.488) (width 0.25) (layer "B.Cu") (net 2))
 (segment (start 148.082 90.17) (end 144.9096 93.3424) (width 0.25) (layer "B.Cu") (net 2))
 (segment (start 113.1897 100.7509) (end 112.9175 101.0231) (width 0.25) (layer "B.Cu") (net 2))
 (segment (start 112.9175 101.0231) (end 112.9175 108.5233) (width 0.25) (layer "B.Cu") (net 2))
 (segment (start 116.6322 93.3424) (end 115.4866 94.488) (width 0.25) (layer "B.Cu") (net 2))
 (segment (start 144.9096 93.3424) (end 116.6322 93.3424) (width 0.25) (layer "B.Cu") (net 2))
 (segment (start 112.9175 108.5233) (end 121.92 117.5258) (width 0.25) (layer "B.Cu") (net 2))
 (segment (start 114.4597 90.4349) (end 111.9197 92.9749) (width 0.25) (layer "F.Cu") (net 24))
 (segment (start 114.4597 89.408) (end 114.4597 90.4349) (width 0.25) (layer "F.Cu") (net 24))
 (segment (start 111.9197 92.9749) (end 111.9197 99.674) (width 0.25) (layer "F.Cu") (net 24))
 (segment (start 110.6497 89.1649) (end 110.6497 99.674) (width 0.25) (layer "F.Cu") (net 33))
 (segment (start 114.4597 84.328) (end 114.4597 85.3549) (width 0.25) (layer "F.Cu") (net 33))
 (segment (start 114.4597 85.3549) (end 110.6497 89.1649) (width 0.25) (layer "F.Cu") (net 33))
 (segment (start 134.2858 71.12) (end 125.2289 80.1769) (width 0.25) (layer "B.Cu") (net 33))
 (segment (start 152.654 64.77) (end 146.304 71.12) (width 0.25) (layer "B.Cu") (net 33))
 (segment (start 114.4597 84.328) (end 115.4866 84.328) (width 0.25) (layer "B.Cu") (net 33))
 (segment (start 125.2289 80.1769) (end 119.6377 80.1769) (width 0.25) (layer "B.Cu") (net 33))
 (segment (start 119.6377 80.1769) (end 115.4866 84.328) (width 0.25) (layer "B.Cu") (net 33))
 (segment (start 146.304 71.12) (end 134.2858 71.12) (width 0.25) (layer "B.Cu") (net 33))
 (segment (start 131.6687 70.2007) (end 131.6687 75.9032) (width 0.25) (layer "F.Cu") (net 25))
 (segment (start 125.6112 81.9607) (end 125.6112 101.3705) (width 0.25) (layer "F.Cu") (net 25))
 (segment (start 130.048 68.58) (end 131.6687 70.2007) (width 0.25) (layer "F.Cu") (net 25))
 (segment (start 125.6112 101.3705) (end 119.5397 107.442) (width 0.25) (layer "F.Cu") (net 25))
 (segment (start 131.6687 75.9032) (end 125.6112 81.9607) (width 0.25) (layer "F.Cu") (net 25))
 (segment (start 119.5397 107.442) (end 119.5397 112.014) (width 0.25) (layer "F.Cu") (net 25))
 (segment (start 114.4597 113.0409) (end 114.3 113.2006) (width 0.25) (layer "F.Cu") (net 9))
 (segment (start 130.4475 64.77) (end 129.7194 64.77) (width 0.25) (layer "F.Cu") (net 9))
 (segment (start 137.414 52.07) (end 131.1749 58.3091) (width 0.25) (layer "F.Cu") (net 9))
 (segment (start 131.1749 58.3091) (end 131.1749 64.0426) (width 0.25) (layer "F.Cu") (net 9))
 (segment (start 129.3951 73.007) (end 130.048 73.66) (width 0.25) (layer "F.Cu") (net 9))
 (segment (start 114.4597 112.014) (end 114.4597 110.9871) (width 0.25) (layer "F.Cu") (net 9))
 (segment (start 116.9997 108.4471) (end 114.4597 110.9871) (width 0.25) (layer "F.Cu") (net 9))
 (segment (start 116.9997 85.4024) (end 116.9997 108.4471) (width 0.25) (layer "F.Cu") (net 9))
 (segment (start 114.3 113.2006) (end 114.3 117.5258) (width 0.25) (layer "F.Cu") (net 9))
 (segment (start 129.3951 73.007) (end 116.9997 85.4024) (width 0.25) (layer "F.Cu") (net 9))
 (segment (start 128.4407 66.0487) (end 128.4407 72.0527) (width 0.25) (layer "F.Cu") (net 9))
 (segment (start 129.7194 64.77) (end 128.4407 66.0487) (width 0.25) (layer "F.Cu") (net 9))
 (segment (start 128.4407 72.0527) (end 129.3951 73.007) (width 0.25) (layer "F.Cu") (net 9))
 (segment (start 131.1749 64.0426) (end 130.4475 64.77) (width 0.25) (layer "F.Cu") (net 9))
 (segment (start 114.4597 112.014) (end 114.4597 113.0409) (width 0.25) (layer "F.Cu") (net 9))
 (segment (start 114.3 117.5258) (end 115.4269 117.5258) (width 0.25) (layer "B.Cu") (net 9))
 (segment (start 115.4269 117.8076) (end 115.4269 117.5258) (width 0.25) (layer "B.Cu") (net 9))
 (segment (start 116.272 118.6527) (end 115.4269 117.8076) (width 0.25) (layer "B.Cu") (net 9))
 (segment (start 130.9531 118.6527) (end 116.272 118.6527) (width 0.25) (layer "B.Cu") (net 9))
 (segment (start 132.08 117.5258) (end 130.9531 118.6527) (width 0.25) (layer "B.Cu") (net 9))
 (segment (start 137.414 85.09) (end 136.7784 85.7256) (width 0.25) (layer "F.Cu") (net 13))
 (segment (start 136.7784 116.3718) (end 136.7784 117.1442) (width 0.25) (layer "F.Cu") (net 13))
 (segment (start 136.7784 116.3718) (end 130.694 116.3718) (width 0.25) (layer "F.Cu") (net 13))
 (segment (start 130.694 116.3718) (end 129.54 117.5258) (width 0.25) (layer "F.Cu") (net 13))
 (segment (start 136.7784 117.1442) (end 137.16 117.5258) (width 0.25) (layer "F.Cu") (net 13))
 (segment (start 136.7784 85.7256) (end 136.7784 116.3718) (width 0.25) (layer "F.Cu") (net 13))
 (segment (start 152.1313 110.1745) (end 144.78 117.5258) (width 0.25) (layer "F.Cu") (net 14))
 (segment (start 152.1313 85.6127) (end 152.1313 110.1745) (width 0.25) (layer "F.Cu") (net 14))
 (segment (start 152.654 85.09) (end 152.1313 85.6127) (width 0.25) (layer "F.Cu") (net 14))
 (segment (start 143.6005 118.7053) (end 135.7995 118.7053) (width 0.25) (layer "B.Cu") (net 14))
 (segment (start 135.7995 118.7053) (end 134.62 117.5258) (width 0.25) (layer "B.Cu") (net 14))
 (segment (start 144.78 117.5258) (end 143.6005 118.7053) (width 0.25) (layer "B.Cu") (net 14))
 (segment (start 131.1075 105.7983) (end 119.38 117.5258) (width 0.25) (layer "F.Cu") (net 10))
 (segment (start 137.414 82.55) (end 131.1075 88.8565) (width 0.25) (layer "F.Cu") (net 10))
 (segment (start 131.1075 88.8565) (end 131.1075 105.7983) (width 0.25) (layer "F.Cu") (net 10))
 (segment (start 141.224 85.852) (end 145.542 90.17) (width 0.25) (layer "B.Cu") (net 3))
 (segment (start 137.414 72.39) (end 141.224 76.2) (width 0.25) (layer "B.Cu") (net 3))
 (segment (start 141.224 76.2) (end 141.224 85.852) (width 0.25) (layer "B.Cu") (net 3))
 (segment (start 141.224 88.392) (end 143.002 90.17) (width 0.25) (layer "F.Cu") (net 4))
 (segment (start 137.414 69.85) (end 141.224 73.66) (width 0.25) (layer "F.Cu") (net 4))
 (segment (start 141.224 73.66) (end 141.224 88.392) (width 0.25) (layer "F.Cu") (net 4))
 (segment (start 149.4244 87.6925) (end 149.4244 105.2577) (width 0.25) (layer "F.Cu") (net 12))
 (segment (start 151.2968 85.8201) (end 149.4244 87.6925) (width 0.25) (layer "F.Cu") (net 12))
 (segment (start 144.2721 115.4937) (end 142.24 117.5258) (width 0.25) (layer "F.Cu") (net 12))
 (segment (start 151.2968 83.9072) (end 151.2968 85.8201) (width 0.25) (layer "F.Cu") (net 12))
 (segment (start 152.654 82.55) (end 151.2968 83.9072) (width 0.25) (layer "F.Cu") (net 12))
 (segment (start 144.2721 110.41) (end 144.2721 115.4937) (width 0.25) (layer "F.Cu") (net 12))
 (segment (start 149.4244 105.2577) (end 144.2721 110.41) (width 0.25) (layer "F.Cu") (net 12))
 (segment (start 128.1711 116.3547) (end 127 117.5258) (width 0.25) (layer "B.Cu") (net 12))
 (segment (start 141.0689 116.3547) (end 128.1711 116.3547) (width 0.25) (layer "B.Cu") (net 12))
 (segment (start 142.24 117.5258) (end 141.0689 116.3547) (width 0.25) (layer "B.Cu") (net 12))
 (segment (start 151.384 80.3799) (end 151.384 78.74) (width 0.25) (layer "B.Cu") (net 11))
 (segment (start 149.2089 90.6599) (end 149.2089 87.9531) (width 0.25) (layer "B.Cu") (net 11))
 (segment (start 113.4178 105.5154) (end 120.4421 98.4911) (width 0.25) (layer "B.Cu") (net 11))
 (segment (start 141.3777 98.4911) (end 149.2089 90.6599) (width 0.25) (layer "B.Cu") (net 11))
 (segment (start 113.4178 107.9017) (end 113.4178 105.5154) (width 0.25) (layer "B.Cu") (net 11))
 (segment (start 120.4421 98.4911) (end 141.3777 98.4911) (width 0.25) (layer "B.Cu") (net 11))
 (segment (start 119.9621 114.446) (end 113.4178 107.9017) (width 0.25) (layer "B.Cu") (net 11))
 (segment (start 148.9335 82.8304) (end 151.384 80.3799) (width 0.25) (layer "B.Cu") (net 11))
 (segment (start 121.3802 114.446) (end 119.9621 114.446) (width 0.25) (layer "B.Cu") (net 11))
 (segment (start 149.2089 87.9531) (end 148.9335 87.6777) (width 0.25) (layer "B.Cu") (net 11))
 (segment (start 148.9335 87.6777) (end 148.9335 82.8304) (width 0.25) (layer "B.Cu") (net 11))
 (segment (start 151.384 78.74) (end 152.654 77.47) (width 0.25) (layer "B.Cu") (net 11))
 (segment (start 124.46 117.5258) (end 121.3802 114.446) (width 0.25) (layer "B.Cu") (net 11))
 (segment (start 152.654 67.31) (end 153.8262 68.4822) (width 0.25) (layer "F.Cu") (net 15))
 (segment (start 140.8795 118.7053) (end 139.7 117.5258) (width 0.25) (layer "F.Cu") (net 15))
 (segment (start 153.8262 68.4822) (end 153.8262 88.8111) (width 0.25) (layer "F.Cu") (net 15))
 (segment (start 153.8262 88.8111) (end 152.5833 90.054) (width 0.25) (layer "F.Cu") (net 15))
 (segment (start 152.5833 90.054) (end 152.5833 110.4372) (width 0.25) (layer "F.Cu") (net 15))
 (segment (start 152.5833 110.4372) (end 146.05 116.9705) (width 0.25) (layer "F.Cu") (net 15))
 (segment (start 145.2606 118.7053) (end 140.8795 118.7053) (width 0.25) (layer "F.Cu") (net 15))
 (segment (start 146.05 117.9159) (end 145.2606 118.7053) (width 0.25) (layer "F.Cu") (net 15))
 (segment (start 146.05 116.9705) (end 146.05 117.9159) (width 0.25) (layer "F.Cu") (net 15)))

